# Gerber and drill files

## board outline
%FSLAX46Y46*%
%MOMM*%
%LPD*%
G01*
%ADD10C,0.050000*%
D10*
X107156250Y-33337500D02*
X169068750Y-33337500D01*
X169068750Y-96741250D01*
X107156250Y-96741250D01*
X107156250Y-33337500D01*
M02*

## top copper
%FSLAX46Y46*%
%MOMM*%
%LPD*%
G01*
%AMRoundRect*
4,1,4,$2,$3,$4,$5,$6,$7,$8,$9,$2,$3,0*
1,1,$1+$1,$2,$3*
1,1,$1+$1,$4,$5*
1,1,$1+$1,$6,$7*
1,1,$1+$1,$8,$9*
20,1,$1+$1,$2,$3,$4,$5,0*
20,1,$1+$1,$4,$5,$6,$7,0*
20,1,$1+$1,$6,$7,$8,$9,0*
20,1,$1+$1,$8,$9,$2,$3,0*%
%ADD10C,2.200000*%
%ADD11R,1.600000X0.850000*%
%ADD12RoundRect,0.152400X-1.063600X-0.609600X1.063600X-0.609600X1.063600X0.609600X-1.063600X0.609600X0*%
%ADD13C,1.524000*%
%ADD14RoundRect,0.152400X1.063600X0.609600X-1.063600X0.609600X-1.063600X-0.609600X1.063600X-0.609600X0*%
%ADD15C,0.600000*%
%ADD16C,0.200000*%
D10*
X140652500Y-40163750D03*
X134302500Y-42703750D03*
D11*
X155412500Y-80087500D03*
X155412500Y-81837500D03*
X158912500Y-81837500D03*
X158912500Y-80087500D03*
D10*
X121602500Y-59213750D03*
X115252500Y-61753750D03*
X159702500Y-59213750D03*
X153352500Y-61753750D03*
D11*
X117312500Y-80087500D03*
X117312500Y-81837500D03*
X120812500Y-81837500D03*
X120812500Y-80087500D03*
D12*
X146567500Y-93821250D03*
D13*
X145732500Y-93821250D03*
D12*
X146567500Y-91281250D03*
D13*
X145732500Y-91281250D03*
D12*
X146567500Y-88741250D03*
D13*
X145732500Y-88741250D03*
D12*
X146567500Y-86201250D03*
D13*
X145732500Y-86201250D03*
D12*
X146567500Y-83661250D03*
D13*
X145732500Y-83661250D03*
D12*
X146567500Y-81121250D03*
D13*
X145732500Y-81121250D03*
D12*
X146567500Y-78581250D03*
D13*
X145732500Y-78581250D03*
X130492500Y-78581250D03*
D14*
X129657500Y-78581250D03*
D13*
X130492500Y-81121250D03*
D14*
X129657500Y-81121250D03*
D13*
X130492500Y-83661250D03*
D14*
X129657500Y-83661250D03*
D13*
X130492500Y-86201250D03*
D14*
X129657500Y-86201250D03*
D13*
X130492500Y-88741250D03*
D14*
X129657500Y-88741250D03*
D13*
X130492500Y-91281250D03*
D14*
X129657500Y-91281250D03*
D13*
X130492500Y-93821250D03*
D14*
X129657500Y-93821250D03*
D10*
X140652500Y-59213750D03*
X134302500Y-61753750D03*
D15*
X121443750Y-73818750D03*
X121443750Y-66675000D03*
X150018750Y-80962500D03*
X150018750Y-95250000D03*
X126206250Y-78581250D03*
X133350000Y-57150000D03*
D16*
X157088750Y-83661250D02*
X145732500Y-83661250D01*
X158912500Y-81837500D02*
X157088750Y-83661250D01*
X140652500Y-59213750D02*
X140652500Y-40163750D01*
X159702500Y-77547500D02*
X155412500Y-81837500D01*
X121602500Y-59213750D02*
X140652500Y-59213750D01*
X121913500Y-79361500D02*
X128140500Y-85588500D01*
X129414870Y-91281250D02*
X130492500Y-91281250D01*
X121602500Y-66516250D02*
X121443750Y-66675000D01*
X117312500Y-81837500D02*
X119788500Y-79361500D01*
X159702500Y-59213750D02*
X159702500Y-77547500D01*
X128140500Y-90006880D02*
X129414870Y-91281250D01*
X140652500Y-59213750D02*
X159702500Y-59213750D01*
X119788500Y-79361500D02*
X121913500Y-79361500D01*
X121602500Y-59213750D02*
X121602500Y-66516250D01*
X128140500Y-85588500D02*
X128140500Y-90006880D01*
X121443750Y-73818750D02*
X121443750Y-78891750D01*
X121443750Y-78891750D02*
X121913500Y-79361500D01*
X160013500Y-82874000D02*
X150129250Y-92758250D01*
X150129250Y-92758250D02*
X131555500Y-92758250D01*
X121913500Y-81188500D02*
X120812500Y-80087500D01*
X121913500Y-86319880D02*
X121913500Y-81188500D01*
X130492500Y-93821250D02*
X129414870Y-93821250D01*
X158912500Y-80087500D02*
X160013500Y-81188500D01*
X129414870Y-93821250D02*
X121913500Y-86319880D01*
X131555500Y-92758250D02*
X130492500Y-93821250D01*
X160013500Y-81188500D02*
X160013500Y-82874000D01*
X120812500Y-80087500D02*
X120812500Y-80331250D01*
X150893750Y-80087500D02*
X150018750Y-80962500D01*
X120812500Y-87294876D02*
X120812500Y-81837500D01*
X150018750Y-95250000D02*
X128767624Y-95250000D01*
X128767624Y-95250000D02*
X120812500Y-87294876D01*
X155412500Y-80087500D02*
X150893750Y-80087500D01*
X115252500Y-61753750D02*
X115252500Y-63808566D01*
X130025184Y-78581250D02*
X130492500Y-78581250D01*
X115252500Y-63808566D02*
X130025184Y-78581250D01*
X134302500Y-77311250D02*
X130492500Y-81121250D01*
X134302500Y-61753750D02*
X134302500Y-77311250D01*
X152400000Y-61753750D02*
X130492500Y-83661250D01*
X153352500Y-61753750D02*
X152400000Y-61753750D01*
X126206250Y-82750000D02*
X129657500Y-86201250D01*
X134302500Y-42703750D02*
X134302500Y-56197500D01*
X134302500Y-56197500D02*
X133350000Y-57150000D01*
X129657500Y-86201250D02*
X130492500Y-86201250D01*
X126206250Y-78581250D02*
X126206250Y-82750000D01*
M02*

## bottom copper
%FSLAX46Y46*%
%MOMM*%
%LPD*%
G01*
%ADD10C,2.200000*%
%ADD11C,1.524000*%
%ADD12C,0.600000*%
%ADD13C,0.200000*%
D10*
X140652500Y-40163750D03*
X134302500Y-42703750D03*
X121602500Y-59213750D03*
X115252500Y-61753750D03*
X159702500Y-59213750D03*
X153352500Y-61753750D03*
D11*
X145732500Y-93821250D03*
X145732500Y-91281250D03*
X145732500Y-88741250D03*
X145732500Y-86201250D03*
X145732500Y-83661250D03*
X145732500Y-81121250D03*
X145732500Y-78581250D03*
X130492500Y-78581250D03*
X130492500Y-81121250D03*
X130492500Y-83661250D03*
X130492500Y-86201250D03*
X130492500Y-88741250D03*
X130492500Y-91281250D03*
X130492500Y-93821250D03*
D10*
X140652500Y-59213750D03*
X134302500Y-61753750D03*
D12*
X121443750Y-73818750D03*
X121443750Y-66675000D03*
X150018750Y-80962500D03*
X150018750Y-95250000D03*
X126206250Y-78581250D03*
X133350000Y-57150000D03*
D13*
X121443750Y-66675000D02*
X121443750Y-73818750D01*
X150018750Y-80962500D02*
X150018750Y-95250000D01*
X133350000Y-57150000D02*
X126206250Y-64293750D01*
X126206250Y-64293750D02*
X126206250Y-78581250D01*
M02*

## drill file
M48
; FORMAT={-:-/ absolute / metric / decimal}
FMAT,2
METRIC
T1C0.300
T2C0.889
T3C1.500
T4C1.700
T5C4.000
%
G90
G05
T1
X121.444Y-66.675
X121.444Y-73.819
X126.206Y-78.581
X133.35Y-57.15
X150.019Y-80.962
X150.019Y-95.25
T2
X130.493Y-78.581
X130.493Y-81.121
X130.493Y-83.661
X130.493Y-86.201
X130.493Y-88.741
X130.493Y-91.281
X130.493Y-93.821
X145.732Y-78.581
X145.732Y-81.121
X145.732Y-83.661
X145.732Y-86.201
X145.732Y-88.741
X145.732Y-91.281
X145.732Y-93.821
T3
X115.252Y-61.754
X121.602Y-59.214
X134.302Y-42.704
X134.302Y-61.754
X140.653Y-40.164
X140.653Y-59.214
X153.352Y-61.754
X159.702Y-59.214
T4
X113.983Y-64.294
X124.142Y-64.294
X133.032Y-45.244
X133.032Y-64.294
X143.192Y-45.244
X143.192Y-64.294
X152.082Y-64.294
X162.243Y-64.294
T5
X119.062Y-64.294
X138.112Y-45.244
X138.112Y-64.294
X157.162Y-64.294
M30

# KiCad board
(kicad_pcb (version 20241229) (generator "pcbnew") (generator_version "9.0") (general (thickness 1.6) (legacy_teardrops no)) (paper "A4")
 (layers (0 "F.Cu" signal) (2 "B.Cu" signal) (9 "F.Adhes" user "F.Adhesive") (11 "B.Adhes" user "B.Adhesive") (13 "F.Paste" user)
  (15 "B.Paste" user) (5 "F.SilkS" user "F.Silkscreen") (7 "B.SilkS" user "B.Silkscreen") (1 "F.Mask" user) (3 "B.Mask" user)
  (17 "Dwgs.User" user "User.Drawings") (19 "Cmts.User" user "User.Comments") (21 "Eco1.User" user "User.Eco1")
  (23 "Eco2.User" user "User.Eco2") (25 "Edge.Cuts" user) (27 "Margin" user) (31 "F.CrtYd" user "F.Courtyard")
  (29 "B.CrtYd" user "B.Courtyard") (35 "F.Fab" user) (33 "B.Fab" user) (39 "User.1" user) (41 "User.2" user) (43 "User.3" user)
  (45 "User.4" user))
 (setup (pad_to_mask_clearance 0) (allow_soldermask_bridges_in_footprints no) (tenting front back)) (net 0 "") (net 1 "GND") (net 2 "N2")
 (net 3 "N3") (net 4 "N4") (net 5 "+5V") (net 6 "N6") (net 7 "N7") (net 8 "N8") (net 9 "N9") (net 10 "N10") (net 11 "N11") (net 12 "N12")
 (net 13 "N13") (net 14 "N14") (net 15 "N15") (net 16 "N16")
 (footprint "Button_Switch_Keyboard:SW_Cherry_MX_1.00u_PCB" (layer "F.Cu") (at 140.6525 40.16375)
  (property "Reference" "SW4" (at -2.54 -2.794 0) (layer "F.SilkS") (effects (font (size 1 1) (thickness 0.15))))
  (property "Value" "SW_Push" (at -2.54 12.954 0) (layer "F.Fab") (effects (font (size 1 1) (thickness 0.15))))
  (pad "" np_thru_hole circle (at -7.62 5.08) (size 1.7 1.7) (drill 1.7) (layers "*.Cu" "*.Mask"))
  (pad "" np_thru_hole circle (at -2.54 5.08) (size 4 4) (drill 4) (layers "*.Cu" "*.Mask"))
  (pad "" np_thru_hole circle (at 2.54 5.08) (size 1.7 1.7) (drill 1.7) (layers "*.Cu" "*.Mask"))
  (pad "1" thru_hole circle (at 0 0) (size 2.2 2.2) (drill 1.5) (layers "*.Cu" "*.Mask") (remove_unused_layers no) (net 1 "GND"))
  (pad "2" thru_hole circle (at -6.35 2.54) (size 2.2 2.2) (drill 1.5) (layers "*.Cu" "*.Mask") (remove_unused_layers no) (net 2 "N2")))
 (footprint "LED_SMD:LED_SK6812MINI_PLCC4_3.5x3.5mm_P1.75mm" (layer "F.Cu") (at 157.1625 80.9625)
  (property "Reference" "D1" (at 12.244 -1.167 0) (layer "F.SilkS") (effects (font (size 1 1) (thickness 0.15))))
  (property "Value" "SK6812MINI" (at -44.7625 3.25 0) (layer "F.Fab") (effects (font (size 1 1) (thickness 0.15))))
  (pad "1" smd rect (at -1.75 -0.875) (size 1.6 0.85) (layers "F.Cu" "F.Mask" "F.Paste") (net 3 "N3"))
  (pad "2" smd rect (at -1.75 0.875) (size 1.6 0.85) (layers "F.Cu" "F.Mask" "F.Paste") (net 1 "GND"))
  (pad "3" smd rect (at 1.75 0.875) (size 1.6 0.85) (layers "F.Cu" "F.Mask" "F.Paste") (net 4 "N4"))
  (pad "4" smd rect (at 1.75 -0.875) (size 1.6 0.85) (layers "F.Cu" "F.Mask" "F.Paste") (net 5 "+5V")))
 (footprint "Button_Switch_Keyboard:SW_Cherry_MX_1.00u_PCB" (layer "F.Cu") (at 121.6025 59.21375)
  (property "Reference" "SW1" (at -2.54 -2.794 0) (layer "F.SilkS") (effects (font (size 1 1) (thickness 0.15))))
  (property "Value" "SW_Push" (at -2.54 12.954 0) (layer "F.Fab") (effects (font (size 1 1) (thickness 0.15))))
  (pad "" np_thru_hole circle (at -7.62 5.08) (size 1.7 1.7) (drill 1.7) (layers "*.Cu" "*.Mask"))
  (pad "" np_thru_hole circle (at -2.54 5.08) (size 4 4) (drill 4) (layers "*.Cu" "*.Mask"))
  (pad "" np_thru_hole circle (at 2.54 5.08) (size 1.7 1.7) (drill 1.7) (layers "*.Cu" "*.Mask"))
  (pad "1" thru_hole circle (at 0 0) (size 2.2 2.2) (drill 1.5) (layers "*.Cu" "*.Mask") (remove_unused_layers no) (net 1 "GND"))
  (pad "2" thru_hole circle (at -6.35 2.54) (size 2.2 2.2) (drill 1.5) (layers "*.Cu" "*.Mask") (remove_unused_layers no) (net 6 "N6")))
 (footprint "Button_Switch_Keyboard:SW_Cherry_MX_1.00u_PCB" (layer "F.Cu") (at 159.7025 59.21375)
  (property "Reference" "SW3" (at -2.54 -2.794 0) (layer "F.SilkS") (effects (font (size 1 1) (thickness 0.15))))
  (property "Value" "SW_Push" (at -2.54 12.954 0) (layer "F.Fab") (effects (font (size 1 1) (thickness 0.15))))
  (pad "" np_thru_hole circle (at -7.62 5.08) (size 1.7 1.7) (drill 1.7) (layers "*.Cu" "*.Mask"))
  (pad "" np_thru_hole circle (at -2.54 5.08) (size 4 4) (drill 4) (layers "*.Cu" "*.Mask"))
  (pad "" np_thru_hole circle (at 2.54 5.08) (size 1.7 1.7) (drill 1.7) (layers "*.Cu" "*.Mask"))
  (pad "1" thru_hole circle (at 0 0) (size 2.2 2.2) (drill 1.5) (layers "*.Cu" "*.Mask") (remove_unused_layers no) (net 1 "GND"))
  (pad "2" thru_hole circle (at -6.35 2.54) (size 2.2 2.2) (drill 1.5) (layers "*.Cu" "*.Mask") (remove_unused_layers no) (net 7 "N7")))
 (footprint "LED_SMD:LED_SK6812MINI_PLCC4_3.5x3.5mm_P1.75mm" (layer "F.Cu") (at 119.0625 80.9625)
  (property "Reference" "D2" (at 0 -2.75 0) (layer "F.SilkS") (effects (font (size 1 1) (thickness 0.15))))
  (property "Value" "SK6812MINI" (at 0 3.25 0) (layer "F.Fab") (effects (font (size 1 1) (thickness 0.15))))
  (pad "1" smd rect (at -1.75 -0.875) (size 1.6 0.85) (layers "F.Cu" "F.Mask" "F.Paste") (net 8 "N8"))
  (pad "2" smd rect (at -1.75 0.875) (size 1.6 0.85) (layers "F.Cu" "F.Mask" "F.Paste") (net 1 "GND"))
  (pad "3" smd rect (at 1.75 0.875) (size 1.6 0.85) (layers "F.Cu" "F.Mask" "F.Paste") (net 3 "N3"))
  (pad "4" smd rect (at 1.75 -0.875) (size 1.6 0.85) (layers "F.Cu" "F.Mask" "F.Paste") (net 5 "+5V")))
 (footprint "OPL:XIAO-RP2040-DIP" (layer "F.Cu") (at 138.1125 86.20125 180)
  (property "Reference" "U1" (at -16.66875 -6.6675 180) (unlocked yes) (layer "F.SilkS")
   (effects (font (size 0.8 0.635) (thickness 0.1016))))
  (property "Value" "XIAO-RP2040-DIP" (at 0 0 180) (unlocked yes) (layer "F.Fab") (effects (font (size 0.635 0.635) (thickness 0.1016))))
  (pad "1" smd roundrect (at -8.455 -7.62) (size 2.432 1.524) (layers "F.Cu" "F.Mask") (roundrect_rratio 0.1) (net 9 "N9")
   (thermal_bridge_angle 45))
  (pad "1" thru_hole circle (at -7.62 -7.62) (size 1.524 1.524) (drill 0.889) (layers "*.Cu" "*.Mask") (remove_unused_layers no)
   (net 9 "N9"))
  (pad "2" smd roundrect (at -8.455 -5.08) (size 2.432 1.524) (layers "F.Cu" "F.Mask") (roundrect_rratio 0.1) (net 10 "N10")
   (thermal_bridge_angle 45))
  (pad "2" thru_hole circle (at -7.62 -5.08) (size 1.524 1.524) (drill 0.889) (layers "*.Cu" "*.Mask") (remove_unused_layers no)
   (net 10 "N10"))
  (pad "3" smd roundrect (at -8.455 -2.54) (size 2.432 1.524) (layers "F.Cu" "F.Mask") (roundrect_rratio 0.1) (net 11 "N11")
   (thermal_bridge_angle 45))
  (pad "3" thru_hole circle (at -7.62 -2.54) (size 1.524 1.524) (drill 0.889) (layers "*.Cu" "*.Mask") (remove_unused_layers no)
   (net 11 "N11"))
  (pad "4" smd roundrect (at -8.455 0) (size 2.432 1.524) (layers "F.Cu" "F.Mask") (roundrect_rratio 0.1) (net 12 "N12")
   (thermal_bridge_angle 45))
  (pad "4" thru_hole circle (at -7.62 0) (size 1.524 1.524) (drill 0.889) (layers "*.Cu" "*.Mask") (remove_unused_layers no) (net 12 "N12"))
  (pad "5" smd roundrect (at -8.455 2.54) (size 2.432 1.524) (layers "F.Cu" "F.Mask") (roundrect_rratio 0.1) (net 4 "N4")
   (thermal_bridge_angle 45))
  (pad "5" thru_hole circle (at -7.62 2.54) (size 1.524 1.524) (drill 0.889) (layers "*.Cu" "*.Mask") (remove_unused_layers no) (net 4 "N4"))
  (pad "6" smd roundrect (at -8.455 5.08) (size 2.432 1.524) (layers "F.Cu" "F.Mask") (roundrect_rratio 0.1) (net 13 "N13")
   (thermal_bridge_angle 45))
  (pad "6" thru_hole circle (at -7.62 5.08) (size 1.524 1.524) (drill 0.889) (layers "*.Cu" "*.Mask") (remove_unused_layers no)
   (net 13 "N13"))
  (pad "7" smd roundrect (at -8.455 7.62) (size 2.432 1.524) (layers "F.Cu" "F.Mask") (roundrect_rratio 0.1) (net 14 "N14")
   (thermal_bridge_angle 45))
  (pad "7" thru_hole circle (at -7.62 7.62) (size 1.524 1.524) (drill 0.889) (layers "*.Cu" "*.Mask") (remove_unused_layers no)
   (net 14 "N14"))
  (pad "8" thru_hole circle (at 7.62 7.62 180) (size 1.524 1.524) (drill 0.889) (layers "*.Cu" "*.Mask") (remove_unused_layers no)
   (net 6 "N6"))
  (pad "8" smd roundrect (at 8.455 7.62 180) (size 2.432 1.524) (layers "F.Cu" "F.Mask") (roundrect_rratio 0.1) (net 6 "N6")
   (thermal_bridge_angle 45))
  (pad "9" thru_hole circle (at 7.62 5.08 180) (size 1.524 1.524) (drill 0.889) (layers "*.Cu" "*.Mask") (remove_unused_layers no)
   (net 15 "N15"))
  (pad "9" smd roundrect (at 8.455 5.08 180) (size 2.432 1.524) (layers "F.Cu" "F.Mask") (roundrect_rratio 0.1) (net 15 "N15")
   (thermal_bridge_angle 45))
  (pad "10" thru_hole circle (at 7.62 2.54 180) (size 1.524 1.524) (drill 0.889) (layers "*.Cu" "*.Mask") (remove_unused_layers no)
   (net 7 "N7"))
  (pad "10" smd roundrect (at 8.455 2.54 180) (size 2.432 1.524) (layers "F.Cu" "F.Mask") (roundrect_rratio 0.1) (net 7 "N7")
   (thermal_bridge_angle 45))
  (pad "11" thru_hole circle (at 7.62 0 180) (size 1.524 1.524) (drill 0.889) (layers "*.Cu" "*.Mask") (remove_unused_layers no)
   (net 2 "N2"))
  (pad "11" smd roundrect (at 8.455 0 180) (size 2.432 1.524) (layers "F.Cu" "F.Mask") (roundrect_rratio 0.1) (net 2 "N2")
   (thermal_bridge_angle 45))
  (pad "12" thru_hole circle (at 7.62 -2.54 180) (size 1.524 1.524) (drill 0.889) (layers "*.Cu" "*.Mask") (remove_unused_layers no)
   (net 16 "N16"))
  (pad "12" smd roundrect (at 8.455 -2.54 180) (size 2.432 1.524) (layers "F.Cu" "F.Mask") (roundrect_rratio 0.1) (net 16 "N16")
   (thermal_bridge_angle 45))
  (pad "13" thru_hole circle (at 7.62 -5.08 180) (size 1.524 1.524) (drill 0.889) (layers "*.Cu" "*.Mask") (remove_unused_layers no)
   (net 1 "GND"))
  (pad "13" smd roundrect (at 8.455 -5.08 180) (size 2.432 1.524) (layers "F.Cu" "F.Mask") (roundrect_rratio 0.1) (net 1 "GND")
   (thermal_bridge_angle 45))
  (pad "14" thru_hole circle (at 7.62 -7.62 180) (size 1.524 1.524) (drill 0.889) (layers "*.Cu" "*.Mask") (remove_unused_layers no)
   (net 5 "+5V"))
  (pad "14" smd roundrect (at 8.455 -7.62 180) (size 2.432 1.524) (layers "F.Cu" "F.Mask") (roundrect_rratio 0.1) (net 5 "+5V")
   (thermal_bridge_angle 45)))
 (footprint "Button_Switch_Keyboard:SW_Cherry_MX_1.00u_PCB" (layer "F.Cu") (at 140.6525 59.21375)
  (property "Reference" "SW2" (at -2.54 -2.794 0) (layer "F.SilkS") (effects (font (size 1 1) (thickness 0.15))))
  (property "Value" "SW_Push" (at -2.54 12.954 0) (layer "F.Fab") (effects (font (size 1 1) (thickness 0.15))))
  (pad "" np_thru_hole circle (at -7.62 5.08) (size 1.7 1.7) (drill 1.7) (layers "*.Cu" "*.Mask"))
  (pad "" np_thru_hole circle (at -2.54 5.08) (size 4 4) (drill 4) (layers "*.Cu" "*.Mask"))
  (pad "" np_thru_hole circle (at 2.54 5.08) (size 1.7 1.7) (drill 1.7) (layers "*.Cu" "*.Mask"))
  (pad "1" thru_hole circle (at 0 0) (size 2.2 2.2) (drill 1.5) (layers "*.Cu" "*.Mask") (remove_unused_layers no) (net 1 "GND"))
  (pad "2" thru_hole circle (at -6.35 2.54) (size 2.2 2.2) (drill 1.5) (layers "*.Cu" "*.Mask") (remove_unused_layers no) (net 15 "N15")))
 (gr_rect (start 107.15625 33.3375) (end 169.06875 96.74125) (stroke (width 0.05) (type default)) (fill no) (layer "Edge.Cuts"))
 (segment (start 157.08875 83.66125) (end 145.7325 83.66125) (width 0.2) (layer "F.Cu") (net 4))
 (segment (start 158.9125 81.8375) (end 157.08875 83.66125) (width 0.2) (layer "F.Cu") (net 4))
 (segment (start 140.6525 59.21375) (end 140.6525 40.16375) (width 0.2) (layer "F.Cu") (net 1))
 (segment (start 159.7025 77.5475) (end 155.4125 81.8375) (width 0.2) (layer "F.Cu") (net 1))
 (segment (start 121.6025 59.21375) (end 140.6525 59.21375) (width 0.2) (layer "F.Cu") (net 1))
 (segment (start 121.9135 79.3615) (end 128.1405 85.5885) (width 0.2) (layer "F.Cu") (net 1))
 (segment (start 129.41487 91.28125) (end 130.4925 91.28125) (width 0.2) (layer "F.Cu") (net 1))
 (segment (start 121.6025 66.51625) (end 121.44375 66.675) (width 0.2) (layer "F.Cu") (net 1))
 (segment (start 117.3125 81.8375) (end 119.7885 79.3615) (width 0.2) (layer "F.Cu") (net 1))
 (segment (start 159.7025 59.21375) (end 159.7025 77.5475) (width 0.2) (layer "F.Cu") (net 1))
 (segment (start 128.1405 90.00688) (end 129.41487 91.28125) (width 0.2) (layer "F.Cu") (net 1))
 (segment (start 140.6525 59.21375) (end 159.7025 59.21375) (width 0.2) (layer "F.Cu") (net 1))
 (segment (start 119.7885 79.3615) (end 121.9135 79.3615) (width 0.2) (layer "F.Cu") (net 1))
 (segment (start 121.6025 59.21375) (end 121.6025 66.51625) (width 0.2) (layer "F.Cu") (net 1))
 (segment (start 128.1405 85.5885) (end 128.1405 90.00688) (width 0.2) (layer "F.Cu") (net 1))
 (segment (start 121.44375 73.81875) (end 121.44375 78.89175) (width 0.2) (layer "F.Cu") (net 1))
 (segment (start 121.44375 78.89175) (end 121.9135 79.3615) (width 0.2) (layer "F.Cu") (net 1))
 (via (at 121.44375 73.81875) (size 0.6) (drill 0.3) (layers "F.Cu" "B.Cu") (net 1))
 (via (at 121.44375 66.675) (size 0.6) (drill 0.3) (layers "F.Cu" "B.Cu") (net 1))
 (segment (start 121.44375 66.675) (end 121.44375 73.81875) (width 0.2) (layer "B.Cu") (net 1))
 (segment (start 160.0135 82.874) (end 150.12925 92.75825) (width 0.2) (layer "F.Cu") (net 5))
 (segment (start 150.12925 92.75825) (end 131.5555 92.75825) (width 0.2) (layer "F.Cu") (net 5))
 (segment (start 121.9135 81.1885) (end 120.8125 80.0875) (width 0.2) (layer "F.Cu") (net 5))
 (segment (start 121.9135 86.31988) (end 121.9135 81.1885) (width 0.2) (layer "F.Cu") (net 5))
 (segment (start 130.4925 93.82125) (end 129.41487 93.82125) (width 0.2) (layer "F.Cu") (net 5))
 (segment (start 158.9125 80.0875) (end 160.0135 81.1885) (width 0.2) (layer "F.Cu") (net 5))
 (segment (start 129.41487 93.82125) (end 121.9135 86.31988) (width 0.2) (layer "F.Cu") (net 5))
 (segment (start 131.5555 92.75825) (end 130.4925 93.82125) (width 0.2) (layer "F.Cu") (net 5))
 (segment (start 160.0135 81.1885) (end 160.0135 82.874) (width 0.2) (layer "F.Cu") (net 5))
 (segment (start 120.8125 80.0875) (end 120.8125 80.33125) (width 0.2) (layer "F.Cu") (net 5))
 (segment (start 150.89375 80.0875) (end 150.01875 80.9625) (width 0.2) (layer "F.Cu") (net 3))
 (segment (start 120.8125 87.294876) (end 120.8125 81.8375) (width 0.2) (layer "F.Cu") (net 3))
 (segment (start 150.01875 95.25) (end 128.767624 95.25) (width 0.2) (layer "F.Cu") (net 3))
 (segment (start 128.767624 95.25) (end 120.8125 87.294876) (width 0.2) (layer "F.Cu") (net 3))
 (segment (start 155.4125 80.0875) (end 150.89375 80.0875) (width 0.2) (layer "F.Cu") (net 3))
 (via (at 150.01875 80.9625) (size 0.6) (drill 0.3) (layers "F.Cu" "B.Cu") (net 3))
 (via (at 150.01875 95.25) (size 0.6) (drill 0.3) (layers "F.Cu" "B.Cu") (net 3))
 (segment (start 150.01875 80.9625) (end 150.01875 95.25) (width 0.2) (layer "B.Cu") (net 3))
 (segment (start 115.2525 61.75375) (end 115.2525 63.808566) (width 0.2) (layer "F.Cu") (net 6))
 (segment (start 130.025184 78.58125) (end 130.4925 78.58125) (width 0.2) (layer "F.Cu") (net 6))
 (segment (start 115.2525 63.808566) (end 130.025184 78.58125) (width 0.2) (layer "F.Cu") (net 6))
 (segment (start 134.3025 77.31125) (end 130.4925 81.12125) (width 0.2) (layer "F.Cu") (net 15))
 (segment (start 134.3025 61.75375) (end 134.3025 77.31125) (width 0.2) (layer "F.Cu") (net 15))
 (segment (start 152.4 61.75375) (end 130.4925 83.66125) (width 0.2) (layer "F.Cu") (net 7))
 (segment (start 153.3525 61.75375) (end 152.4 61.75375) (width 0.2) (layer "F.Cu") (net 7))
 (segment (start 126.20625 82.75) (end 129.6575 86.20125) (width 0.2) (layer "F.Cu") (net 2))
 (segment (start 134.3025 42.70375) (end 134.3025 56.1975) (width 0.2) (layer "F.Cu") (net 2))
 (segment (start 134.3025 56.1975) (end 133.35 57.15) (width 0.2) (layer "F.Cu") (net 2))
 (segment (start 129.6575 86.20125) (end 130.4925 86.20125) (width 0.2) (layer "F.Cu") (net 2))
 (segment (start 126.20625 78.58125) (end 126.20625 82.75) (width 0.2) (layer "F.Cu") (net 2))
 (via (at 126.20625 78.58125) (size 0.6) (drill 0.3) (layers "F.Cu" "B.Cu") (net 2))
 (via (at 133.35 57.15) (size 0.6) (drill 0.3) (layers "F.Cu" "B.Cu") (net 2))
 (segment (start 133.35 57.15) (end 126.20625 64.29375) (width 0.2) (layer "B.Cu") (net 2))
 (segment (start 126.20625 64.29375) (end 126.20625 78.58125) (width 0.2) (layer "B.Cu") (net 2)))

